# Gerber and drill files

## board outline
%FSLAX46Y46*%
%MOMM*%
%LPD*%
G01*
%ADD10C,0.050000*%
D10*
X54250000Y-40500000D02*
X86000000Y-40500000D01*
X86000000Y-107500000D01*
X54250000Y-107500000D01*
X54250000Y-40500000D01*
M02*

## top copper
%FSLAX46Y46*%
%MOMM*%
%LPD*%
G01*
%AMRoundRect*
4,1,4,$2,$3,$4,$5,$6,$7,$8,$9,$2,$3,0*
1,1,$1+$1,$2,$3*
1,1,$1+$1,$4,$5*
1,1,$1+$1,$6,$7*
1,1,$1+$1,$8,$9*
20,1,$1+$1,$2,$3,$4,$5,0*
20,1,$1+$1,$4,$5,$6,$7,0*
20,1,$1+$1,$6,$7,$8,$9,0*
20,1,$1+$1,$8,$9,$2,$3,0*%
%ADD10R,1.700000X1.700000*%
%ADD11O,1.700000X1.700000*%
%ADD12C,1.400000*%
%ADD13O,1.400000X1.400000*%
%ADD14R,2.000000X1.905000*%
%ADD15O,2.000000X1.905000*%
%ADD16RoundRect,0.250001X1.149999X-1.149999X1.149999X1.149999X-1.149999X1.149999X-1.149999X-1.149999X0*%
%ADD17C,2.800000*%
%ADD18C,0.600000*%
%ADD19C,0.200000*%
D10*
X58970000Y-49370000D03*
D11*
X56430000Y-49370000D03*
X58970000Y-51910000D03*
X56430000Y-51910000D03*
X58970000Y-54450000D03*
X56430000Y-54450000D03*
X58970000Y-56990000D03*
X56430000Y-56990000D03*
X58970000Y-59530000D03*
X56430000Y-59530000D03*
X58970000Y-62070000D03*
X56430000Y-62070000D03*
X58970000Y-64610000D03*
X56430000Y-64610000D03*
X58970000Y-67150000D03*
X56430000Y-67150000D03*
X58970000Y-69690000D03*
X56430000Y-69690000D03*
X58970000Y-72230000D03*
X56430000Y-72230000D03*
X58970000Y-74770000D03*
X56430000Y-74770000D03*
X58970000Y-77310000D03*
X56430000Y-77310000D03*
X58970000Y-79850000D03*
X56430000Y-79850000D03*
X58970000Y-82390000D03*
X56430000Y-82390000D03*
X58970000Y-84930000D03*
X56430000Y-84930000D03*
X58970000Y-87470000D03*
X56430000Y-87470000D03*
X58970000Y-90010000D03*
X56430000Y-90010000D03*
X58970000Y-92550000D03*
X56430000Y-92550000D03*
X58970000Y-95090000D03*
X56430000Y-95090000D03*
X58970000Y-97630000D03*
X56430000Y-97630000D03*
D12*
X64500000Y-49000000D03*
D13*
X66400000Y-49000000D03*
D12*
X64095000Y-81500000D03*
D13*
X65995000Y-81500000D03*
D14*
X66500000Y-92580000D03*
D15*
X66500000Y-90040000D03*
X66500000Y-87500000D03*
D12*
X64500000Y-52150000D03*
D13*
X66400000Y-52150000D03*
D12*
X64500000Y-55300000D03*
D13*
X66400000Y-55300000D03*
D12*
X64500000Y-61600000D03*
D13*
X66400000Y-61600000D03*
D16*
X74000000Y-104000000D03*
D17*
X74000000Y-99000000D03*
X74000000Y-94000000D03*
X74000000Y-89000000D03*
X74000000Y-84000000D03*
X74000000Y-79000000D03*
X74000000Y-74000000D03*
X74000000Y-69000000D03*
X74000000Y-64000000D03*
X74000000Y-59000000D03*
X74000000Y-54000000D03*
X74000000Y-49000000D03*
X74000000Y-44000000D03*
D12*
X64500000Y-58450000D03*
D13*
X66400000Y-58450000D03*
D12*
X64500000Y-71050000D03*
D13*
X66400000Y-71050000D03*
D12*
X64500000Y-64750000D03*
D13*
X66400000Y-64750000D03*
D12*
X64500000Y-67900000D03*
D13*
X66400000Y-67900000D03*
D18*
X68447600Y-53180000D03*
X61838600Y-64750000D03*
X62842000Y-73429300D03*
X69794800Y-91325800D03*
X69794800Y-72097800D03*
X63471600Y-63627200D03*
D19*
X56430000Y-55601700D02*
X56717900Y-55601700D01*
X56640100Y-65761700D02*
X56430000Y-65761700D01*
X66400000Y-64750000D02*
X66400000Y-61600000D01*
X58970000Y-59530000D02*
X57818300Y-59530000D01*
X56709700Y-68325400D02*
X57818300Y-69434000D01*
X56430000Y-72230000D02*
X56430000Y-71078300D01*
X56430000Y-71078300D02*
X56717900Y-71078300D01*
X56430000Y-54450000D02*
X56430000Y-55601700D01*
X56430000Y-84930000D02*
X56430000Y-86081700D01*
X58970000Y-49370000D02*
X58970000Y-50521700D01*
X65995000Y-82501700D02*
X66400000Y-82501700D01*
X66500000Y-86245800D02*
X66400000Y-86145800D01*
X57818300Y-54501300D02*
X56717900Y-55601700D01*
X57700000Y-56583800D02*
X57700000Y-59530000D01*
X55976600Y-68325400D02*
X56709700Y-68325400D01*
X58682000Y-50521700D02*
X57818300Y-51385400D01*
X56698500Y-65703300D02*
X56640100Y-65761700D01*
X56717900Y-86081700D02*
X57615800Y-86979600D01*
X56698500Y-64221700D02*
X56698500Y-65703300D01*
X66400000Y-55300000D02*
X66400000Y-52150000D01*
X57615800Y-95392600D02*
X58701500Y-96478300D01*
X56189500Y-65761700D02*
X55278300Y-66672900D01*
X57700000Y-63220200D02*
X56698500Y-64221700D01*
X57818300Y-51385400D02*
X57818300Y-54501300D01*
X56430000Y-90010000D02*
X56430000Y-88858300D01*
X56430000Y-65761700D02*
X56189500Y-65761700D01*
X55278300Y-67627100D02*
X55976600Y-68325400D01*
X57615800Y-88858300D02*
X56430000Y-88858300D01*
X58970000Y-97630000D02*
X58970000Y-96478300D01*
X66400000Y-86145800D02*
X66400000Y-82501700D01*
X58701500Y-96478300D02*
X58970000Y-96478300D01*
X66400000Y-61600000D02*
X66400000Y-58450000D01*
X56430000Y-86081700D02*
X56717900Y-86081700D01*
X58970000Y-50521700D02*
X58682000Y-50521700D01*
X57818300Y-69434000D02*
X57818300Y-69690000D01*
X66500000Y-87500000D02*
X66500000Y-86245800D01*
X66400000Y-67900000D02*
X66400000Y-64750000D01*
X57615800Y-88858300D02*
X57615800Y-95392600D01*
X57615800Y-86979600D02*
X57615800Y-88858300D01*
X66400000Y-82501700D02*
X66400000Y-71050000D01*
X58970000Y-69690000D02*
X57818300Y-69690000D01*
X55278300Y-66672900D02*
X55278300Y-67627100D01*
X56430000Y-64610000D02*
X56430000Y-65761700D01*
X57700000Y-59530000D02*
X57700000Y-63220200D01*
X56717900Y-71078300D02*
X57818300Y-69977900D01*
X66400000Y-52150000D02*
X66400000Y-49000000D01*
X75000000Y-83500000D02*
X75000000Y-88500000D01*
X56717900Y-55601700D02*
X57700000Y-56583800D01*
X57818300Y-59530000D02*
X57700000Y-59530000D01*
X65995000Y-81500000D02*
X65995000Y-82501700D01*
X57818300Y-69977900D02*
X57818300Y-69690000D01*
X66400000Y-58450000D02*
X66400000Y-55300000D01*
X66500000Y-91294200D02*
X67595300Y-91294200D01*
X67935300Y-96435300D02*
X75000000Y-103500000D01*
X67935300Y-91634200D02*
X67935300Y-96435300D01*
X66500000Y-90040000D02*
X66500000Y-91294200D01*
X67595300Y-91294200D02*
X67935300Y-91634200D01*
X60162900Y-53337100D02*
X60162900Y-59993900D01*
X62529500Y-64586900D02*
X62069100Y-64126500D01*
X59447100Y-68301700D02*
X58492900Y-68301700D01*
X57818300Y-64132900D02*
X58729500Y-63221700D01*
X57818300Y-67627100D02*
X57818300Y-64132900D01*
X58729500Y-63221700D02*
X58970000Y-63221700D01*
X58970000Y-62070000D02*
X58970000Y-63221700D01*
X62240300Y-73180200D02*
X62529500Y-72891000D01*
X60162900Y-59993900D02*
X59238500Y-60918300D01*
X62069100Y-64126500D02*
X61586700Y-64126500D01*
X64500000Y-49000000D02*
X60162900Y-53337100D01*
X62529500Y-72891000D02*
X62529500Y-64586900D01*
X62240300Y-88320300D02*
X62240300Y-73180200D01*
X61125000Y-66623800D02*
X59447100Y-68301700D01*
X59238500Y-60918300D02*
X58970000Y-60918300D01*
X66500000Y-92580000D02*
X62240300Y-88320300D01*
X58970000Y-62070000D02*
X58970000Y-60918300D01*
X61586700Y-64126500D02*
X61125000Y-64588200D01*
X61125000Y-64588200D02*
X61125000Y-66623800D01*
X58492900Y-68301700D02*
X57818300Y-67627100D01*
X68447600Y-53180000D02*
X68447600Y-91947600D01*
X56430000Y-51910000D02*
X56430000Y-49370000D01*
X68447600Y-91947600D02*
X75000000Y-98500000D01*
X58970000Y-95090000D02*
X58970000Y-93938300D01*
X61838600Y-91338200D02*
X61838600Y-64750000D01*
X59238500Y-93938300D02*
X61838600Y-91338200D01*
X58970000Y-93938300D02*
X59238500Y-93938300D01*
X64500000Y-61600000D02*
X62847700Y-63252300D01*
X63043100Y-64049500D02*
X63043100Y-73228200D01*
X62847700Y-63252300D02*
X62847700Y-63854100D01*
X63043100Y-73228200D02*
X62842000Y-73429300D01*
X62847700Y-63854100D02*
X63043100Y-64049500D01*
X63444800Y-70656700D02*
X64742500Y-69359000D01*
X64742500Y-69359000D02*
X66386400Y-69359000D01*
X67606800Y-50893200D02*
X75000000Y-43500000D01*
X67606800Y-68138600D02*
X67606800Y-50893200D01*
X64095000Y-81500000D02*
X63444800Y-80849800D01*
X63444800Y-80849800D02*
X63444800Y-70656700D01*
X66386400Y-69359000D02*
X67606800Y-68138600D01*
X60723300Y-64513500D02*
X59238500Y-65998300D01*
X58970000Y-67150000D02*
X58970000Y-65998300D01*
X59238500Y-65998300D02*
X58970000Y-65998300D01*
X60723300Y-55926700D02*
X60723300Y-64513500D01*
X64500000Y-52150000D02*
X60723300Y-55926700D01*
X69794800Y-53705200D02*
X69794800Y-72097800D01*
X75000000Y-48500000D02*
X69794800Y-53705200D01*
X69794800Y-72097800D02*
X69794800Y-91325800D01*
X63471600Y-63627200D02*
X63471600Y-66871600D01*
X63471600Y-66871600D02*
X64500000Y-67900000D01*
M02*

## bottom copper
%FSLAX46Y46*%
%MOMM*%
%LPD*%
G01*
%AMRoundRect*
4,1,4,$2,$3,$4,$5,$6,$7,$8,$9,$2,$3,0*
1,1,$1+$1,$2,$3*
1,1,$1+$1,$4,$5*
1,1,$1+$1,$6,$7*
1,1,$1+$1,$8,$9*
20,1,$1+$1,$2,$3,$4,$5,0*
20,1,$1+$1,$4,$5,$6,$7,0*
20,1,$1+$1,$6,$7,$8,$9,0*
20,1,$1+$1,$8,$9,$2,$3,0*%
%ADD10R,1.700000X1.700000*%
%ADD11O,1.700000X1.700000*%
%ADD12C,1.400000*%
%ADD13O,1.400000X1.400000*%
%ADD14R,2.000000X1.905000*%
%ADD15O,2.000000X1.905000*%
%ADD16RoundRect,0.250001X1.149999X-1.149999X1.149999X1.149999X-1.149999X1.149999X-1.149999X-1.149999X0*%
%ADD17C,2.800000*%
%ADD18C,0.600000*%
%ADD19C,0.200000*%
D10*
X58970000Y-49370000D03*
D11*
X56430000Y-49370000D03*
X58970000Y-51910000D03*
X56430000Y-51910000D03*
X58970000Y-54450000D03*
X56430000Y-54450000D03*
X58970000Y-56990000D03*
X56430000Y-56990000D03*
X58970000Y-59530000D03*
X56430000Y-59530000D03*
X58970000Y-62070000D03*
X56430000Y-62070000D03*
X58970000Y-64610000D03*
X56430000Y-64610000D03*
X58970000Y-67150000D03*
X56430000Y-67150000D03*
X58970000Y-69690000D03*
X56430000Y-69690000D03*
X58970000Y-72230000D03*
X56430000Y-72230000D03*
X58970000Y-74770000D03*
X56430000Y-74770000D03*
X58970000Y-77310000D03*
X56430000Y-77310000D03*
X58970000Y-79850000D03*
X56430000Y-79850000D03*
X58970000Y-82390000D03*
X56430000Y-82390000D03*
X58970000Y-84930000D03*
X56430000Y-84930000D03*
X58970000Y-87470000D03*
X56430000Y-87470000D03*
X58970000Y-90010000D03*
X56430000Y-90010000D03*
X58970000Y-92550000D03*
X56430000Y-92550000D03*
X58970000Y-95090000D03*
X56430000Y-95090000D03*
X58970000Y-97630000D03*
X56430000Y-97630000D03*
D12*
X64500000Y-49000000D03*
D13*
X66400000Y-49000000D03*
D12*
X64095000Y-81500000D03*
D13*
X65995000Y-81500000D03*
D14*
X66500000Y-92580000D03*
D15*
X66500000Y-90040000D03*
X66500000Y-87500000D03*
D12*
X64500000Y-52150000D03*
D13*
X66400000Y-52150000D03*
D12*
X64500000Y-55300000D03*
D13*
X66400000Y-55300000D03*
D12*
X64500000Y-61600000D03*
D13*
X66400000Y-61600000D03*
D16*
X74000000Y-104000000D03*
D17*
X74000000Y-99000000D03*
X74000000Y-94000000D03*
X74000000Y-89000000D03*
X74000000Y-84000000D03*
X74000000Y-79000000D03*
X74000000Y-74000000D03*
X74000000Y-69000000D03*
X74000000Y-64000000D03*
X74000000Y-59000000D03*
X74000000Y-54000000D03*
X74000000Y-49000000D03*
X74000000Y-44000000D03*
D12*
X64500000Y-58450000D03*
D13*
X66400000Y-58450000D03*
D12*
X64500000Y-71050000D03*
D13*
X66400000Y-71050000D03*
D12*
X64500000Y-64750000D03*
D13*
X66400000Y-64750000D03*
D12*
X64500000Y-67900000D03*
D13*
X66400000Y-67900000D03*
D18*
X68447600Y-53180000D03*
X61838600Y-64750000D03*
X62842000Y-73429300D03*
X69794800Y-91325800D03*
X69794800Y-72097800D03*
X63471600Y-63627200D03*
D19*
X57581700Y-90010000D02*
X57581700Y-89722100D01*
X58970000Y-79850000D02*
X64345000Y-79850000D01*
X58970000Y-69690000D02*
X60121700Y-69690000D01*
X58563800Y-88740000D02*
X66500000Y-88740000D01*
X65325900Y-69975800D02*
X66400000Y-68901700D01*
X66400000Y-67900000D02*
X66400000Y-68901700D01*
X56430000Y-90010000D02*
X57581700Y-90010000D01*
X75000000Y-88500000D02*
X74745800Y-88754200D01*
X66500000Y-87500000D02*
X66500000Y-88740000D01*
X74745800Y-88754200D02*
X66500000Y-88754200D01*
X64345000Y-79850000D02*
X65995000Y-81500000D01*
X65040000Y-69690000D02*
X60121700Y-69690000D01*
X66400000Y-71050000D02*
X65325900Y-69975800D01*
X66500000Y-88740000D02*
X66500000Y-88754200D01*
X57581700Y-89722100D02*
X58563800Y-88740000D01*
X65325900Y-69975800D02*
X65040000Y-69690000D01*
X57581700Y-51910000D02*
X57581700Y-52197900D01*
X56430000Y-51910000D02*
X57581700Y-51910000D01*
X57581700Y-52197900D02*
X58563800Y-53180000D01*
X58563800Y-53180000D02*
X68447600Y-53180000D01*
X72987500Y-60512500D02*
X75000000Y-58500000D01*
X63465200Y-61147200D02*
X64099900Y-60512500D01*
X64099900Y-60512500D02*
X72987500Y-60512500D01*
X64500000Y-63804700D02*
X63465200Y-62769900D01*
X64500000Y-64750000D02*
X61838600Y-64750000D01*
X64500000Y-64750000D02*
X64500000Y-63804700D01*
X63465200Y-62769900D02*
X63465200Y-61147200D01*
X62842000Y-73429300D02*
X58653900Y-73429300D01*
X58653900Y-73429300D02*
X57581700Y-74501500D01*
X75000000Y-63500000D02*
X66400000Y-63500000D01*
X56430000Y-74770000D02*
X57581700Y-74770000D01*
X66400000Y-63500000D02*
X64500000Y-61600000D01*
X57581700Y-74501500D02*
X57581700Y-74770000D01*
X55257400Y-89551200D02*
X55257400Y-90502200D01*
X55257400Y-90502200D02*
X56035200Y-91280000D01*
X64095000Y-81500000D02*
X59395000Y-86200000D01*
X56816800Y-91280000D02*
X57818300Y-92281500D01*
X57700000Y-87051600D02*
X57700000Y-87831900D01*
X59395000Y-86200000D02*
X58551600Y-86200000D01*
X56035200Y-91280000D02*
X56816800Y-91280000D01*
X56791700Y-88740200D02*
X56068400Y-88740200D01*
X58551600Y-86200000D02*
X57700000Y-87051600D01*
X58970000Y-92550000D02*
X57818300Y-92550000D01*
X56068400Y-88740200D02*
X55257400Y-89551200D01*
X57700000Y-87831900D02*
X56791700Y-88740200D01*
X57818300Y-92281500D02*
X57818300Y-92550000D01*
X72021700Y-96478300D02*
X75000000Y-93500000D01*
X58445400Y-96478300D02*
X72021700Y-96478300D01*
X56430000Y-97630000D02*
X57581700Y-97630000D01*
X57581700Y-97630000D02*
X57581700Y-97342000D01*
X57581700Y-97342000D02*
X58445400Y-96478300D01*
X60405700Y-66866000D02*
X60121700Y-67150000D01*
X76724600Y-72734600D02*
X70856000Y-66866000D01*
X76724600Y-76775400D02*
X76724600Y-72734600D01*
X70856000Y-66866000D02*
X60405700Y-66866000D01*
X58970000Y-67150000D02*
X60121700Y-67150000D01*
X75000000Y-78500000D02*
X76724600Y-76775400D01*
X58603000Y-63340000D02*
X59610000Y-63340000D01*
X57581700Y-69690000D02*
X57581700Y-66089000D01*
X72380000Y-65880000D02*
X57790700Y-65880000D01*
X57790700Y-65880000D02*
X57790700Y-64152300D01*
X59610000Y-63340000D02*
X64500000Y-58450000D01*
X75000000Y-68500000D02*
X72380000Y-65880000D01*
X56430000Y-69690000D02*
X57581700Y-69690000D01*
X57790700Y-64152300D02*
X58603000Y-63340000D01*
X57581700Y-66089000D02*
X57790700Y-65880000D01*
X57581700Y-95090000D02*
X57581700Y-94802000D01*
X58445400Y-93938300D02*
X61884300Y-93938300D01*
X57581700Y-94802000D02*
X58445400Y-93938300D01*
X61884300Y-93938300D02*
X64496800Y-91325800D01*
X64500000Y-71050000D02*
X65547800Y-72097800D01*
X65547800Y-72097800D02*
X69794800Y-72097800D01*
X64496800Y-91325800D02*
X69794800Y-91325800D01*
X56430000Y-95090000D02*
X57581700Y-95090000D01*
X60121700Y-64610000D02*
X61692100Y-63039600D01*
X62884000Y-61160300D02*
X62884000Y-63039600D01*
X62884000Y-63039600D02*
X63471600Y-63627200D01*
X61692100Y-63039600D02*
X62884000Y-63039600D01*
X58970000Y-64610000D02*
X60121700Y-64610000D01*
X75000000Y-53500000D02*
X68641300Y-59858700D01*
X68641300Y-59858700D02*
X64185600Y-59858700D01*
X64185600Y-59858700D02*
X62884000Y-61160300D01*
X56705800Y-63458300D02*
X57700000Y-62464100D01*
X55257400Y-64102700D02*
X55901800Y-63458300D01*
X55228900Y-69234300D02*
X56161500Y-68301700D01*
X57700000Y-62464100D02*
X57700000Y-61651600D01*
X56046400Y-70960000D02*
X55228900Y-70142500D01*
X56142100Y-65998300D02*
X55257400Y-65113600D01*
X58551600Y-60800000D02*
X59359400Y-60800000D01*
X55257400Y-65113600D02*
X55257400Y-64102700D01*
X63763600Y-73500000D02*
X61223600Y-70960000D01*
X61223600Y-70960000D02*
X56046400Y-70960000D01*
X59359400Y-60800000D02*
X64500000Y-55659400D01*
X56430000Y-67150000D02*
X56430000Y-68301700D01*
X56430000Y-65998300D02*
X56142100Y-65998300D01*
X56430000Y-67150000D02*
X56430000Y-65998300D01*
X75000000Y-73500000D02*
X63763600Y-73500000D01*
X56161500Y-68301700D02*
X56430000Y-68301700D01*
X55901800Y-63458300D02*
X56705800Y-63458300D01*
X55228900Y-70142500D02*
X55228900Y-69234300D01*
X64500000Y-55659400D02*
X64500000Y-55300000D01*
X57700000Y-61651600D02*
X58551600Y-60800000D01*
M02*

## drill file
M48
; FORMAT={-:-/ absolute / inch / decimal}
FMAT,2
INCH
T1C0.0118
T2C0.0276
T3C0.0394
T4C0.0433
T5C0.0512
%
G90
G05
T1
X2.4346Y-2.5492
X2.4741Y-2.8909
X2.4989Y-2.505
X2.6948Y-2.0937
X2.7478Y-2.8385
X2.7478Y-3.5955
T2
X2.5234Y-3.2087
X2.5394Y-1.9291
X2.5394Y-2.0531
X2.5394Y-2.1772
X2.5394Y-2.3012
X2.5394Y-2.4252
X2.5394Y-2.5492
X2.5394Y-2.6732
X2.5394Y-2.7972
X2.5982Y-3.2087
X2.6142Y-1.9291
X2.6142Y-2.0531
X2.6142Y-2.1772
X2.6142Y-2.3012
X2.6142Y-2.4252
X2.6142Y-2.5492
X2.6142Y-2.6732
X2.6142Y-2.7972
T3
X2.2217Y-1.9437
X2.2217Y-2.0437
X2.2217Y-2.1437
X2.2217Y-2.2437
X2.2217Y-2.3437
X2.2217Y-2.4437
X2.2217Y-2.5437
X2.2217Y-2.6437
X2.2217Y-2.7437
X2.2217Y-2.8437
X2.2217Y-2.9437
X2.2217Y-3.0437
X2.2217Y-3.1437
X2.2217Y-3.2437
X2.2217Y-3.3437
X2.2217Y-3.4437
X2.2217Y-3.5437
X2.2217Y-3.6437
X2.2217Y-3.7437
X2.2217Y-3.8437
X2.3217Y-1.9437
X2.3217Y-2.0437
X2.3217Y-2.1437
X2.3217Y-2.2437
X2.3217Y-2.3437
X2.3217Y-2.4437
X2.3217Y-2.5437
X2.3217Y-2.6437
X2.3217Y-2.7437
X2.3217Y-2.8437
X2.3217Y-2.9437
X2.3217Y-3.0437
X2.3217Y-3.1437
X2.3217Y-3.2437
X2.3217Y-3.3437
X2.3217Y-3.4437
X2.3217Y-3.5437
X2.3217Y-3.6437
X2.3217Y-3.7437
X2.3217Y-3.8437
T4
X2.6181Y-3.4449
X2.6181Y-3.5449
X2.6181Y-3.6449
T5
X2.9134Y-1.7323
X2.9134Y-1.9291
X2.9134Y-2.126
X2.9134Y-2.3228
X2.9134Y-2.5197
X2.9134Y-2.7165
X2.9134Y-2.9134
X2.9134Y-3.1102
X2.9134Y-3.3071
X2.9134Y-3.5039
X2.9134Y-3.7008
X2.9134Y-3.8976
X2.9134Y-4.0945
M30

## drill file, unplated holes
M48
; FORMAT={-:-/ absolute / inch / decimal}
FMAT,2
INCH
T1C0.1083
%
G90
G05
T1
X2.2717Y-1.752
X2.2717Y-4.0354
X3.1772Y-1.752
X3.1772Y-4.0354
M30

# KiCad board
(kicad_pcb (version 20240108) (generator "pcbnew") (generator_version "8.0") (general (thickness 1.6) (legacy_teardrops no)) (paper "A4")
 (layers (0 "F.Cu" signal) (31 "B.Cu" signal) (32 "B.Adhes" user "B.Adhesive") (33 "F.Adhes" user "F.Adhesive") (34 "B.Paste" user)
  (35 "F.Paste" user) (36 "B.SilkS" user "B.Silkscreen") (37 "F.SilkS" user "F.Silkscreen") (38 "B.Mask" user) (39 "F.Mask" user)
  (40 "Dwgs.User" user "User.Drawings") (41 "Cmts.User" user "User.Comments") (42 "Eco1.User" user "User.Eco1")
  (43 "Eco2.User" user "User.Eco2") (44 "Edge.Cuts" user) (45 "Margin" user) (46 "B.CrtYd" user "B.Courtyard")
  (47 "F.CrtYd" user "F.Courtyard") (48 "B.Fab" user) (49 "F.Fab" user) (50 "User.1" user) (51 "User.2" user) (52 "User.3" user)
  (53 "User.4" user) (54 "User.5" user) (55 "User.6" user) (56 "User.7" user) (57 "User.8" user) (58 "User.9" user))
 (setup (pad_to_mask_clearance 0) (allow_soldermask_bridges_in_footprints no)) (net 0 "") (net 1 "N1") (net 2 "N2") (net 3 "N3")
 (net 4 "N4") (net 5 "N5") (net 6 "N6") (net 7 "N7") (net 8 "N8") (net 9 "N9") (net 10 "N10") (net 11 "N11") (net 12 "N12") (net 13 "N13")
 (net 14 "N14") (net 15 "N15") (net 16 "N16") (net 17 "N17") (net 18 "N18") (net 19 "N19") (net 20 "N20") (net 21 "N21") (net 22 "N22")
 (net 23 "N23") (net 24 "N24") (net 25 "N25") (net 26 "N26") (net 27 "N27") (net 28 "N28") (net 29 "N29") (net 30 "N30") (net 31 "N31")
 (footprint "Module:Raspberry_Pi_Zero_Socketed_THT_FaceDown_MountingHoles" (layer "F.Cu") (at 58.97 49.37)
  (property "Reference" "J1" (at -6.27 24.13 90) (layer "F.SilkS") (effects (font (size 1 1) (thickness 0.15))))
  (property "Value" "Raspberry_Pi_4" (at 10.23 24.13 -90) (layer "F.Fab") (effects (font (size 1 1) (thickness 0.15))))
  (pad "" np_thru_hole circle (at -1.27 -4.87 90) (size 2.75 2.75) (drill 2.75) (layers "*.Cu" "*.Mask") (solder_mask_margin 1.625))
  (pad "" np_thru_hole circle (at -1.27 53.13 90) (size 2.75 2.75) (drill 2.75) (layers "*.Cu" "*.Mask") (solder_mask_margin 1.625))
  (pad "" np_thru_hole circle (at 21.73 -4.87 90) (size 2.75 2.75) (drill 2.75) (layers "*.Cu" "*.Mask") (solder_mask_margin 1.625))
  (pad "" np_thru_hole circle (at 21.73 53.13 90) (size 2.75 2.75) (drill 2.75) (layers "*.Cu" "*.Mask") (solder_mask_margin 1.625))
  (pad "1" thru_hole rect (at 0 0) (size 1.7 1.7) (drill 1) (layers "*.Cu" "*.Mask") (remove_unused_layers no) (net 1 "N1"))
  (pad "2" thru_hole oval (at -2.54 0) (size 1.7 1.7) (drill 1) (layers "*.Cu" "*.Mask") (remove_unused_layers no) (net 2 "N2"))
  (pad "3" thru_hole oval (at 0 2.54) (size 1.7 1.7) (drill 1) (layers "*.Cu" "*.Mask") (remove_unused_layers no) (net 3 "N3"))
  (pad "4" thru_hole oval (at -2.54 2.54) (size 1.7 1.7) (drill 1) (layers "*.Cu" "*.Mask") (remove_unused_layers no) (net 2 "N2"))
  (pad "5" thru_hole oval (at 0 5.08) (size 1.7 1.7) (drill 1) (layers "*.Cu" "*.Mask") (remove_unused_layers no) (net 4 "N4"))
  (pad "6" thru_hole oval (at -2.54 5.08) (size 1.7 1.7) (drill 1) (layers "*.Cu" "*.Mask") (remove_unused_layers no) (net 1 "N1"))
  (pad "7" thru_hole oval (at 0 7.62) (size 1.7 1.7) (drill 1) (layers "*.Cu" "*.Mask") (remove_unused_layers no) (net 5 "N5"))
  (pad "8" thru_hole oval (at -2.54 7.62) (size 1.7 1.7) (drill 1) (layers "*.Cu" "*.Mask") (remove_unused_layers no) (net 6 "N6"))
  (pad "9" thru_hole oval (at 0 10.16) (size 1.7 1.7) (drill 1) (layers "*.Cu" "*.Mask") (remove_unused_layers no) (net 1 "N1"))
  (pad "10" thru_hole oval (at -2.54 10.16) (size 1.7 1.7) (drill 1) (layers "*.Cu" "*.Mask") (remove_unused_layers no) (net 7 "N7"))
  (pad "11" thru_hole oval (at 0 12.7) (size 1.7 1.7) (drill 1) (layers "*.Cu" "*.Mask") (remove_unused_layers no) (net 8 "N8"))
  (pad "12" thru_hole oval (at -2.54 12.7) (size 1.7 1.7) (drill 1) (layers "*.Cu" "*.Mask") (remove_unused_layers no) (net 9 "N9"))
  (pad "13" thru_hole oval (at 0 15.24) (size 1.7 1.7) (drill 1) (layers "*.Cu" "*.Mask") (remove_unused_layers no) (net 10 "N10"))
  (pad "14" thru_hole oval (at -2.54 15.24) (size 1.7 1.7) (drill 1) (layers "*.Cu" "*.Mask") (remove_unused_layers no) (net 1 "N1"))
  (pad "15" thru_hole oval (at 0 17.78) (size 1.7 1.7) (drill 1) (layers "*.Cu" "*.Mask") (remove_unused_layers no) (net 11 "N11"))
  (pad "16" thru_hole oval (at -2.54 17.78) (size 1.7 1.7) (drill 1) (layers "*.Cu" "*.Mask") (remove_unused_layers no) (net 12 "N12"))
  (pad "17" thru_hole oval (at 0 20.32) (size 1.7 1.7) (drill 1) (layers "*.Cu" "*.Mask") (remove_unused_layers no) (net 1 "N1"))
  (pad "18" thru_hole oval (at -2.54 20.32) (size 1.7 1.7) (drill 1) (layers "*.Cu" "*.Mask") (remove_unused_layers no) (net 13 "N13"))
  (pad "19" thru_hole oval (at 0 22.86) (size 1.7 1.7) (drill 1) (layers "*.Cu" "*.Mask") (remove_unused_layers no) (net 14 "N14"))
  (pad "20" thru_hole oval (at -2.54 22.86) (size 1.7 1.7) (drill 1) (layers "*.Cu" "*.Mask") (remove_unused_layers no) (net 1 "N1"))
  (pad "21" thru_hole oval (at 0 25.4) (size 1.7 1.7) (drill 1) (layers "*.Cu" "*.Mask") (remove_unused_layers no) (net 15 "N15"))
  (pad "22" thru_hole oval (at -2.54 25.4) (size 1.7 1.7) (drill 1) (layers "*.Cu" "*.Mask") (remove_unused_layers no) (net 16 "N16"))
  (pad "23" thru_hole oval (at 0 27.94) (size 1.7 1.7) (drill 1) (layers "*.Cu" "*.Mask") (remove_unused_layers no) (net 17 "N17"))
  (pad "24" thru_hole oval (at -2.54 27.94) (size 1.7 1.7) (drill 1) (layers "*.Cu" "*.Mask") (remove_unused_layers no) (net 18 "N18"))
  (pad "25" thru_hole oval (at 0 30.48) (size 1.7 1.7) (drill 1) (layers "*.Cu" "*.Mask") (remove_unused_layers no) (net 1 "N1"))
  (pad "26" thru_hole oval (at -2.54 30.48) (size 1.7 1.7) (drill 1) (layers "*.Cu" "*.Mask") (remove_unused_layers no) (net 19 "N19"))
  (pad "27" thru_hole oval (at 0 33.02) (size 1.7 1.7) (drill 1) (layers "*.Cu" "*.Mask") (remove_unused_layers no) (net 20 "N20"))
  (pad "28" thru_hole oval (at -2.54 33.02) (size 1.7 1.7) (drill 1) (layers "*.Cu" "*.Mask") (remove_unused_layers no) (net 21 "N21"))
  (pad "29" thru_hole oval (at 0 35.56) (size 1.7 1.7) (drill 1) (layers "*.Cu" "*.Mask") (remove_unused_layers no) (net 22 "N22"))
  (pad "30" thru_hole oval (at -2.54 35.56) (size 1.7 1.7) (drill 1) (layers "*.Cu" "*.Mask") (remove_unused_layers no) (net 1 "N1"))
  (pad "31" thru_hole oval (at 0 38.1) (size 1.7 1.7) (drill 1) (layers "*.Cu" "*.Mask") (remove_unused_layers no) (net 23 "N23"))
  (pad "32" thru_hole oval (at -2.54 38.1) (size 1.7 1.7) (drill 1) (layers "*.Cu" "*.Mask") (remove_unused_layers no) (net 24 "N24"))
  (pad "33" thru_hole oval (at 0 40.64) (size 1.7 1.7) (drill 1) (layers "*.Cu" "*.Mask") (remove_unused_layers no) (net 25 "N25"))
  (pad "34" thru_hole oval (at -2.54 40.64) (size 1.7 1.7) (drill 1) (layers "*.Cu" "*.Mask") (remove_unused_layers no) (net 1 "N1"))
  (pad "35" thru_hole oval (at 0 43.18) (size 1.7 1.7) (drill 1) (layers "*.Cu" "*.Mask") (remove_unused_layers no) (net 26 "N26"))
  (pad "36" thru_hole oval (at -2.54 43.18) (size 1.7 1.7) (drill 1) (layers "*.Cu" "*.Mask") (remove_unused_layers no) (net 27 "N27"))
  (pad "37" thru_hole oval (at 0 45.72) (size 1.7 1.7) (drill 1) (layers "*.Cu" "*.Mask") (remove_unused_layers no) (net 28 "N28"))
  (pad "38" thru_hole oval (at -2.54 45.72) (size 1.7 1.7) (drill 1) (layers "*.Cu" "*.Mask") (remove_unused_layers no) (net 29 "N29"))
  (pad "39" thru_hole oval (at 0 48.26) (size 1.7 1.7) (drill 1) (layers "*.Cu" "*.Mask") (remove_unused_layers no) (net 1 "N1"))
  (pad "40" thru_hole oval (at -2.54 48.26) (size 1.7 1.7) (drill 1) (layers "*.Cu" "*.Mask") (remove_unused_layers no) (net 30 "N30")))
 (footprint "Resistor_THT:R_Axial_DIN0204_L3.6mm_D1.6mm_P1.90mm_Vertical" (layer "F.Cu") (at 64.5 49)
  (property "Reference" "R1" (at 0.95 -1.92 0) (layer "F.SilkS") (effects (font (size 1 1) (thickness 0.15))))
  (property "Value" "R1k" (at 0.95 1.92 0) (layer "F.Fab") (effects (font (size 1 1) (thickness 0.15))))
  (pad "1" thru_hole circle (at 0 0) (size 1.4 1.4) (drill 0.7) (layers "*.Cu" "*.Mask") (remove_unused_layers no) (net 8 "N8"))
  (pad "2" thru_hole oval (at 1.9 0) (size 1.4 1.4) (drill 0.7) (layers "*.Cu" "*.Mask") (remove_unused_layers no) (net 1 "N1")))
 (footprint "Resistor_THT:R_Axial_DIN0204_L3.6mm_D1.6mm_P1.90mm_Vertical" (layer "F.Cu") (at 64.095 81.5)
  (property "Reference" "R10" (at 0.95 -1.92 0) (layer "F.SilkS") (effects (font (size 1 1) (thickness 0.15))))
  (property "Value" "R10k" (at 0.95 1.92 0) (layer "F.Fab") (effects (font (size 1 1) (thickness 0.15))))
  (pad "1" thru_hole circle (at 0 0) (size 1.4 1.4) (drill 0.7) (layers "*.Cu" "*.Mask") (remove_unused_layers no) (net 26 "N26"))
  (pad "2" thru_hole oval (at 1.9 0) (size 1.4 1.4) (drill 0.7) (layers "*.Cu" "*.Mask") (remove_unused_layers no) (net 1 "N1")))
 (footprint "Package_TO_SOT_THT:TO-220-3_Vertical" (layer "F.Cu") (at 66.5 92.58 90)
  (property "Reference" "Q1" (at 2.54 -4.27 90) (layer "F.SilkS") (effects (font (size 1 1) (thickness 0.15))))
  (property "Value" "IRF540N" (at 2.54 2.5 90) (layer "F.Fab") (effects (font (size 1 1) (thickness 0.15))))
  (pad "1" thru_hole rect (at 0 0 90) (size 1.905 2) (drill 1.1) (layers "*.Cu" "*.Mask") (remove_unused_layers no) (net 8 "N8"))
  (pad "2" thru_hole oval (at 2.54 0 90) (size 1.905 2) (drill 1.1) (layers "*.Cu" "*.Mask") (remove_unused_layers no) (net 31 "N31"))
  (pad "3" thru_hole oval (at 5.08 0 90) (size 1.905 2) (drill 1.1) (layers "*.Cu" "*.Mask") (remove_unused_layers no) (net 1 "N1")))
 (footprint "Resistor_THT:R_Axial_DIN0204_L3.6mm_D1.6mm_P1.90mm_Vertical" (layer "F.Cu") (at 64.5 52.15)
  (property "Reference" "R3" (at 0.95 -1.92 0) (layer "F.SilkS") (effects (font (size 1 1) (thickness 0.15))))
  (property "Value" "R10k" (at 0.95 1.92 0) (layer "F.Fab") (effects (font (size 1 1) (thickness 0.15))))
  (pad "1" thru_hole circle (at 0 0) (size 1.4 1.4) (drill 0.7) (layers "*.Cu" "*.Mask") (remove_unused_layers no) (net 11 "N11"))
  (pad "2" thru_hole oval (at 1.9 0) (size 1.4 1.4) (drill 0.7) (layers "*.Cu" "*.Mask") (remove_unused_layers no) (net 1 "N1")))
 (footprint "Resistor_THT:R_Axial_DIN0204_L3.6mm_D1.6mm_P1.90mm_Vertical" (layer "F.Cu") (at 64.5 55.3)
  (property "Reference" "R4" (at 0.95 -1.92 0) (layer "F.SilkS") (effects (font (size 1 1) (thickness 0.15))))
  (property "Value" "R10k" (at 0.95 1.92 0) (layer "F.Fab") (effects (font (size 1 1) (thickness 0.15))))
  (pad "1" thru_hole circle (at 0 0) (size 1.4 1.4) (drill 0.7) (layers "*.Cu" "*.Mask") (remove_unused_layers no) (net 12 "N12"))
  (pad "2" thru_hole oval (at 1.9 0) (size 1.4 1.4) (drill 0.7) (layers "*.Cu" "*.Mask") (remove_unused_layers no) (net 1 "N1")))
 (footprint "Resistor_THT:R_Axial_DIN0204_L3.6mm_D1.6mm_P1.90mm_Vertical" (layer "F.Cu") (at 64.5 61.6)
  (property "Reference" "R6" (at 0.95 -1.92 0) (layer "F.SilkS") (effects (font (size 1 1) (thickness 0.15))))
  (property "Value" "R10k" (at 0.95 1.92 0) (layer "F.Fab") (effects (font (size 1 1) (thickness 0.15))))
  (pad "1" thru_hole circle (at 0 0) (size 1.4 1.4) (drill 0.7) (layers "*.Cu" "*.Mask") (remove_unused_layers no) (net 16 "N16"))
  (pad "2" thru_hole oval (at 1.9 0) (size 1.4 1.4) (drill 0.7) (layers "*.Cu" "*.Mask") (remove_unused_layers no) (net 1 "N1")))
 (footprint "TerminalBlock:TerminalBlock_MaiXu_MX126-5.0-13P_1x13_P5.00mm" (layer "F.Cu") (at 74 104 90)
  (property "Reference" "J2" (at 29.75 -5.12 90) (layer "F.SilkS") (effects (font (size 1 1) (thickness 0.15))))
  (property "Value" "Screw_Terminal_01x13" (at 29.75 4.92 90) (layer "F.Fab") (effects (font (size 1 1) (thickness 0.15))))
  (pad "1" thru_hole roundrect (at 0 0 90) (size 2.8 2.8) (drill 1.3) (layers "*.Cu" "*.Mask") (remove_unused_layers no)
   (roundrect_rratio 0.089286) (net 31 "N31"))
  (pad "2" thru_hole circle (at 5 0 90) (size 2.8 2.8) (drill 1.3) (layers "*.Cu" "*.Mask") (remove_unused_layers no) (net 2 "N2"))
  (pad "3" thru_hole circle (at 10 0 90) (size 2.8 2.8) (drill 1.3) (layers "*.Cu" "*.Mask") (remove_unused_layers no) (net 30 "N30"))
  (pad "4" thru_hole circle (at 15 0 90) (size 2.8 2.8) (drill 1.3) (layers "*.Cu" "*.Mask") (remove_unused_layers no) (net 1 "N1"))
  (pad "5" thru_hole circle (at 20 0 90) (size 2.8 2.8) (drill 1.3) (layers "*.Cu" "*.Mask") (remove_unused_layers no) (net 1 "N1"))
  (pad "6" thru_hole circle (at 25 0 90) (size 2.8 2.8) (drill 1.3) (layers "*.Cu" "*.Mask") (remove_unused_layers no) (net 11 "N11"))
  (pad "7" thru_hole circle (at 30 0 90) (size 2.8 2.8) (drill 1.3) (layers "*.Cu" "*.Mask") (remove_unused_layers no) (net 12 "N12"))
  (pad "8" thru_hole circle (at 35 0 90) (size 2.8 2.8) (drill 1.3) (layers "*.Cu" "*.Mask") (remove_unused_layers no) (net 13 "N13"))
  (pad "9" thru_hole circle (at 40 0 90) (size 2.8 2.8) (drill 1.3) (layers "*.Cu" "*.Mask") (remove_unused_layers no) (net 16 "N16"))
  (pad "10" thru_hole circle (at 45 0 90) (size 2.8 2.8) (drill 1.3) (layers "*.Cu" "*.Mask") (remove_unused_layers no) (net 28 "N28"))
  (pad "11" thru_hole circle (at 50 0 90) (size 2.8 2.8) (drill 1.3) (layers "*.Cu" "*.Mask") (remove_unused_layers no) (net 10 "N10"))
  (pad "12" thru_hole circle (at 55 0 90) (size 2.8 2.8) (drill 1.3) (layers "*.Cu" "*.Mask") (remove_unused_layers no) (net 29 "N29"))
  (pad "13" thru_hole circle (at 60 0 90) (size 2.8 2.8) (drill 1.3) (layers "*.Cu" "*.Mask") (remove_unused_layers no) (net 26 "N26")))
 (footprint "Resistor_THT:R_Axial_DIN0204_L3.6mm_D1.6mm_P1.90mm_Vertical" (layer "F.Cu") (at 64.5 58.45)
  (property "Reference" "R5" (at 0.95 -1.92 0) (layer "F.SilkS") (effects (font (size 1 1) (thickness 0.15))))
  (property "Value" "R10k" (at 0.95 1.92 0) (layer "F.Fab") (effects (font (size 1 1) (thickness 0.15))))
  (pad "1" thru_hole circle (at 0 0) (size 1.4 1.4) (drill 0.7) (layers "*.Cu" "*.Mask") (remove_unused_layers no) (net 13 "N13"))
  (pad "2" thru_hole oval (at 1.9 0) (size 1.4 1.4) (drill 0.7) (layers "*.Cu" "*.Mask") (remove_unused_layers no) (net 1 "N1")))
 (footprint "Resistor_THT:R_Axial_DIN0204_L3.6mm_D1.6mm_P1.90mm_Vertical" (layer "F.Cu") (at 64.5 71.05)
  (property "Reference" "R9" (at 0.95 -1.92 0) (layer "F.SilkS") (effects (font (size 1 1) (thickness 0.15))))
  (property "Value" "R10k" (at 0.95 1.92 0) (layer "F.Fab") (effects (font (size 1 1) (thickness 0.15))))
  (pad "1" thru_hole circle (at 0 0) (size 1.4 1.4) (drill 0.7) (layers "*.Cu" "*.Mask") (remove_unused_layers no) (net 29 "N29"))
  (pad "2" thru_hole oval (at 1.9 0) (size 1.4 1.4) (drill 0.7) (layers "*.Cu" "*.Mask") (remove_unused_layers no) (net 1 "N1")))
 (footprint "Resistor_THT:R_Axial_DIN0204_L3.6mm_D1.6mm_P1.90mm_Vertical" (layer "F.Cu") (at 64.5 64.75)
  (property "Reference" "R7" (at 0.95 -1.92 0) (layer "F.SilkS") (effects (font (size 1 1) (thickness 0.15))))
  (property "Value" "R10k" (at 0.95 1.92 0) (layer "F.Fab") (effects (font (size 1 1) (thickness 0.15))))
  (pad "1" thru_hole circle (at 0 0) (size 1.4 1.4) (drill 0.7) (layers "*.Cu" "*.Mask") (remove_unused_layers no) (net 28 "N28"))
  (pad "2" thru_hole oval (at 1.9 0) (size 1.4 1.4) (drill 0.7) (layers "*.Cu" "*.Mask") (remove_unused_layers no) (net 1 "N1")))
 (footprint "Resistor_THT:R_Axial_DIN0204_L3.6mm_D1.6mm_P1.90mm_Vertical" (layer "F.Cu") (at 64.5 67.9)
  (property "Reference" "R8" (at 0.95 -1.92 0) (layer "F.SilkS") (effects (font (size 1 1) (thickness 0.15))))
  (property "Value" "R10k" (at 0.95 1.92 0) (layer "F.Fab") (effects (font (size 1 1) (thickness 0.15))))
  (pad "1" thru_hole circle (at 0 0) (size 1.4 1.4) (drill 0.7) (layers "*.Cu" "*.Mask") (remove_unused_layers no) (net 10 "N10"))
  (pad "2" thru_hole oval (at 1.9 0) (size 1.4 1.4) (drill 0.7) (layers "*.Cu" "*.Mask") (remove_unused_layers no) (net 1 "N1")))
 (gr_rect (start 54.25 40.5) (end 86 107.5) (stroke (width 0.05) (type default)) (fill none) (layer "Edge.Cuts"))
 (segment (start 56.43 55.6017) (end 56.7179 55.6017) (width 0.2) (layer "F.Cu") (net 1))
 (segment (start 56.6401 65.7617) (end 56.43 65.7617) (width 0.2) (layer "F.Cu") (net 1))
 (segment (start 66.4 64.75) (end 66.4 61.6) (width 0.2) (layer "F.Cu") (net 1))
 (segment (start 58.97 59.53) (end 57.8183 59.53) (width 0.2) (layer "F.Cu") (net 1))
 (segment (start 56.7097 68.3254) (end 57.8183 69.434) (width 0.2) (layer "F.Cu") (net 1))
 (segment (start 56.43 72.23) (end 56.43 71.0783) (width 0.2) (layer "F.Cu") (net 1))
 (segment (start 56.43 71.0783) (end 56.7179 71.0783) (width 0.2) (layer "F.Cu") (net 1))
 (segment (start 56.43 54.45) (end 56.43 55.6017) (width 0.2) (layer "F.Cu") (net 1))
 (segment (start 56.43 84.93) (end 56.43 86.0817) (width 0.2) (layer "F.Cu") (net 1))
 (segment (start 58.97 49.37) (end 58.97 50.5217) (width 0.2) (layer "F.Cu") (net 1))
 (segment (start 65.995 82.5017) (end 66.4 82.5017) (width 0.2) (layer "F.Cu") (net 1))
 (segment (start 66.5 86.2458) (end 66.4 86.1458) (width 0.2) (layer "F.Cu") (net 1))
 (segment (start 57.8183 54.5013) (end 56.7179 55.6017) (width 0.2) (layer "F.Cu") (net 1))
 (segment (start 57.7 56.5838) (end 57.7 59.53) (width 0.2) (layer "F.Cu") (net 1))
 (segment (start 55.9766 68.3254) (end 56.7097 68.3254) (width 0.2) (layer "F.Cu") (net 1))
 (segment (start 58.682 50.5217) (end 57.8183 51.3854) (width 0.2) (layer "F.Cu") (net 1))
 (segment (start 56.6985 65.7033) (end 56.6401 65.7617) (width 0.2) (layer "F.Cu") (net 1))
 (segment (start 56.7179 86.0817) (end 57.6158 86.9796) (width 0.2) (layer "F.Cu") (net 1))
 (segment (start 56.6985 64.2217) (end 56.6985 65.7033) (width 0.2) (layer "F.Cu") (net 1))
 (segment (start 66.4 55.3) (end 66.4 52.15) (width 0.2) (layer "F.Cu") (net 1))
 (segment (start 57.6158 95.3926) (end 58.7015 96.4783) (width 0.2) (layer "F.Cu") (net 1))
 (segment (start 56.1895 65.7617) (end 55.2783 66.6729) (width 0.2) (layer "F.Cu") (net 1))
 (segment (start 57.7 63.2202) (end 56.6985 64.2217) (width 0.2) (layer "F.Cu") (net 1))
 (segment (start 57.8183 51.3854) (end 57.8183 54.5013) (width 0.2) (layer "F.Cu") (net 1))
 (segment (start 56.43 90.01) (end 56.43 88.8583) (width 0.2) (layer "F.Cu") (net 1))
 (segment (start 56.43 65.7617) (end 56.1895 65.7617) (width 0.2) (layer "F.Cu") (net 1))
 (segment (start 55.2783 67.6271) (end 55.9766 68.3254) (width 0.2) (layer "F.Cu") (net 1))
 (segment (start 57.6158 88.8583) (end 56.43 88.8583) (width 0.2) (layer "F.Cu") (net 1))
 (segment (start 58.97 97.63) (end 58.97 96.4783) (width 0.2) (layer "F.Cu") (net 1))
 (segment (start 66.4 86.1458) (end 66.4 82.5017) (width 0.2) (layer "F.Cu") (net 1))
 (segment (start 58.7015 96.4783) (end 58.97 96.4783) (width 0.2) (layer "F.Cu") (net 1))
 (segment (start 66.4 61.6) (end 66.4 58.45) (width 0.2) (layer "F.Cu") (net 1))
 (segment (start 56.43 86.0817) (end 56.7179 86.0817) (width 0.2) (layer "F.Cu") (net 1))
 (segment (start 58.97 50.5217) (end 58.682 50.5217) (width 0.2) (layer "F.Cu") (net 1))
 (segment (start 57.8183 69.434) (end 57.8183 69.69) (width 0.2) (layer "F.Cu") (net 1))
 (segment (start 66.5 87.5) (end 66.5 86.2458) (width 0.2) (layer "F.Cu") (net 1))
 (segment (start 66.4 67.9) (end 66.4 64.75) (width 0.2) (layer "F.Cu") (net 1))
 (segment (start 57.6158 88.8583) (end 57.6158 95.3926) (width 0.2) (layer "F.Cu") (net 1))
 (segment (start 57.6158 86.9796) (end 57.6158 88.8583) (width 0.2) (layer "F.Cu") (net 1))
 (segment (start 66.4 82.5017) (end 66.4 71.05) (width 0.2) (layer "F.Cu") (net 1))
 (segment (start 58.97 69.69) (end 57.8183 69.69) (width 0.2) (layer "F.Cu") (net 1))
 (segment (start 55.2783 66.6729) (end 55.2783 67.6271) (width 0.2) (layer "F.Cu") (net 1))
 (segment (start 56.43 64.61) (end 56.43 65.7617) (width 0.2) (layer "F.Cu") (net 1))
 (segment (start 57.7 59.53) (end 57.7 63.2202) (width 0.2) (layer "F.Cu") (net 1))
 (segment (start 56.7179 71.0783) (end 57.8183 69.9779) (width 0.2) (layer "F.Cu") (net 1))
 (segment (start 66.4 52.15) (end 66.4 49) (width 0.2) (layer "F.Cu") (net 1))
 (segment (start 75 83.5) (end 75 88.5) (width 0.2) (layer "F.Cu") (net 1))
 (segment (start 56.7179 55.6017) (end 57.7 56.5838) (width 0.2) (layer "F.Cu") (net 1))
 (segment (start 57.8183 59.53) (end 57.7 59.53) (width 0.2) (layer "F.Cu") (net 1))
 (segment (start 65.995 81.5) (end 65.995 82.5017) (width 0.2) (layer "F.Cu") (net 1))
 (segment (start 57.8183 69.9779) (end 57.8183 69.69) (width 0.2) (layer "F.Cu") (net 1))
 (segment (start 66.4 58.45) (end 66.4 55.3) (width 0.2) (layer "F.Cu") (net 1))
 (segment (start 57.5817 90.01) (end 57.5817 89.7221) (width 0.2) (layer "B.Cu") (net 1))
 (segment (start 58.97 79.85) (end 64.345 79.85) (width 0.2) (layer "B.Cu") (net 1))
 (segment (start 58.97 69.69) (end 60.1217 69.69) (width 0.2) (layer "B.Cu") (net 1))
 (segment (start 58.5638 88.74) (end 66.5 88.74) (width 0.2) (layer "B.Cu") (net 1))
 (segment (start 65.3259 69.9758) (end 66.4 68.9017) (width 0.2) (layer "B.Cu") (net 1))
 (segment (start 66.4 67.9) (end 66.4 68.9017) (width 0.2) (layer "B.Cu") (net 1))
 (segment (start 56.43 90.01) (end 57.5817 90.01) (width 0.2) (layer "B.Cu") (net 1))
 (segment (start 75 88.5) (end 74.7458 88.7542) (width 0.2) (layer "B.Cu") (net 1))
 (segment (start 66.5 87.5) (end 66.5 88.74) (width 0.2) (layer "B.Cu") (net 1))
 (segment (start 74.7458 88.7542) (end 66.5 88.7542) (width 0.2) (layer "B.Cu") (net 1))
 (segment (start 64.345 79.85) (end 65.995 81.5) (width 0.2) (layer "B.Cu") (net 1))
 (segment (start 65.04 69.69) (end 60.1217 69.69) (width 0.2) (layer "B.Cu") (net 1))
 (segment (start 66.4 71.05) (end 65.3259 69.9758) (width 0.2) (layer "B.Cu") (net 1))
 (segment (start 66.5 88.74) (end 66.5 88.7542) (width 0.2) (layer "B.Cu") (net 1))
 (segment (start 57.5817 89.7221) (end 58.5638 88.74) (width 0.2) (layer "B.Cu") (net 1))
 (segment (start 65.3259 69.9758) (end 65.04 69.69) (width 0.2) (layer "B.Cu") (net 1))
 (segment (start 66.5 91.2942) (end 67.5953 91.2942) (width 0.2) (layer "F.Cu") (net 31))
 (segment (start 67.9353 96.4353) (end 75 103.5) (width 0.2) (layer "F.Cu") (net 31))
 (segment (start 67.9353 91.6342) (end 67.9353 96.4353) (width 0.2) (layer "F.Cu") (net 31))
 (segment (start 66.5 90.04) (end 66.5 91.2942) (width 0.2) (layer "F.Cu") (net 31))
 (segment (start 67.5953 91.2942) (end 67.9353 91.6342) (width 0.2) (layer "F.Cu") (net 31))
 (segment (start 60.1629 53.3371) (end 60.1629 59.9939) (width 0.2) (layer "F.Cu") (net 8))
 (segment (start 62.5295 64.5869) (end 62.0691 64.1265) (width 0.2) (layer "F.Cu") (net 8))
 (segment (start 59.4471 68.3017) (end 58.4929 68.3017) (width 0.2) (layer "F.Cu") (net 8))
 (segment (start 57.8183 64.1329) (end 58.7295 63.2217) (width 0.2) (layer "F.Cu") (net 8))
 (segment (start 57.8183 67.6271) (end 57.8183 64.1329) (width 0.2) (layer "F.Cu") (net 8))
 (segment (start 58.7295 63.2217) (end 58.97 63.2217) (width 0.2) (layer "F.Cu") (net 8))
 (segment (start 58.97 62.07) (end 58.97 63.2217) (width 0.2) (layer "F.Cu") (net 8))
 (segment (start 62.2403 73.1802) (end 62.5295 72.891) (width 0.2) (layer "F.Cu") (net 8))
 (segment (start 60.1629 59.9939) (end 59.2385 60.9183) (width 0.2) (layer "F.Cu") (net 8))
 (segment (start 62.0691 64.1265) (end 61.5867 64.1265) (width 0.2) (layer "F.Cu") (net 8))
 (segment (start 64.5 49) (end 60.1629 53.3371) (width 0.2) (layer "F.Cu") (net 8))
 (segment (start 62.5295 72.891) (end 62.5295 64.5869) (width 0.2) (layer "F.Cu") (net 8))
 (segment (start 62.2403 88.3203) (end 62.2403 73.1802) (width 0.2) (layer "F.Cu") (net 8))
 (segment (start 61.125 66.6238) (end 59.4471 68.3017) (width 0.2) (layer "F.Cu") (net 8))
 (segment (start 59.2385 60.9183) (end 58.97 60.9183) (width 0.2) (layer "F.Cu") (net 8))
 (segment (start 66.5 92.58) (end 62.2403 88.3203) (width 0.2) (layer "F.Cu") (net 8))
 (segment (start 58.97 62.07) (end 58.97 60.9183) (width 0.2) (layer "F.Cu") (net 8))
 (segment (start 61.5867 64.1265) (end 61.125 64.5882) (width 0.2) (layer "F.Cu") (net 8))
 (segment (start 61.125 64.5882) (end 61.125 66.6238) (width 0.2) (layer "F.Cu") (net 8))
 (segment (start 58.4929 68.3017) (end 57.8183 67.6271) (width 0.2) (layer "F.Cu") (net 8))
 (segment (start 68.4476 53.18) (end 68.4476 91.9476) (width 0.2) (layer "F.Cu") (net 2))
 (segment (start 56.43 51.91) (end 56.43 49.37) (width 0.2) (layer "F.Cu") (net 2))
 (segment (start 68.4476 91.9476) (end 75 98.5) (width 0.2) (layer "F.Cu") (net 2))
 (via (at 68.4476 53.18) (size 0.6) (drill 0.3) (layers "F.Cu" "B.Cu") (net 2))
 (segment (start 57.5817 51.91) (end 57.5817 52.1979) (width 0.2) (layer "B.Cu") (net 2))
 (segment (start 56.43 51.91) (end 57.5817 51.91) (width 0.2) (layer "B.Cu") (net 2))
 (segment (start 57.5817 52.1979) (end 58.5638 53.18) (width 0.2) (layer "B.Cu") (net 2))
 (segment (start 58.5638 53.18) (end 68.4476 53.18) (width 0.2) (layer "B.Cu") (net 2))
 (segment (start 58.97 95.09) (end 58.97 93.9383) (width 0.2) (layer "F.Cu") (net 28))
 (segment (start 61.8386 91.3382) (end 61.8386 64.75) (width 0.2) (layer "F.Cu") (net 28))
 (segment (start 59.2385 93.9383) (end 61.8386 91.3382) (width 0.2) (layer "F.Cu") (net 28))
 (segment (start 58.97 93.9383) (end 59.2385 93.9383) (width 0.2) (layer "F.Cu") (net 28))
 (via (at 61.8386 64.75) (size 0.6) (drill 0.3) (layers "F.Cu" "B.Cu") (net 28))
 (segment (start 72.9875 60.5125) (end 75 58.5) (width 0.2) (layer "B.Cu") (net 28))
 (segment (start 63.4652 61.1472) (end 64.0999 60.5125) (width 0.2) (layer "B.Cu") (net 28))
 (segment (start 64.0999 60.5125) (end 72.9875 60.5125) (width 0.2) (layer "B.Cu") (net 28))
 (segment (start 64.5 63.8047) (end 63.4652 62.7699) (width 0.2) (layer "B.Cu") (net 28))
 (segment (start 64.5 64.75) (end 61.8386 64.75) (width 0.2) (layer "B.Cu") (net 28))
 (segment (start 64.5 64.75) (end 64.5 63.8047) (width 0.2) (layer "B.Cu") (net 28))
 (segment (start 63.4652 62.7699) (end 63.4652 61.1472) (width 0.2) (layer "B.Cu") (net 28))
 (segment (start 64.5 61.6) (end 62.8477 63.2523) (width 0.2) (layer "F.Cu") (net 16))
 (segment (start 63.0431 64.0495) (end 63.0431 73.2282) (width 0.2) (layer "F.Cu") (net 16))
 (segment (start 62.8477 63.2523) (end 62.8477 63.8541) (width 0.2) (layer "F.Cu") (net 16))
 (segment (start 63.0431 73.2282) (end 62.842 73.4293) (width 0.2) (layer "F.Cu") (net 16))
 (segment (start 62.8477 63.8541) (end 63.0431 64.0495) (width 0.2) (layer "F.Cu") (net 16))
 (via (at 62.842 73.4293) (size 0.6) (drill 0.3) (layers "F.Cu" "B.Cu") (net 16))
 (segment (start 62.842 73.4293) (end 58.6539 73.4293) (width 0.2) (layer "B.Cu") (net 16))
 (segment (start 58.6539 73.4293) (end 57.5817 74.5015) (width 0.2) (layer "B.Cu") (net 16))
 (segment (start 75 63.5) (end 66.4 63.5) (width 0.2) (layer "B.Cu") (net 16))
 (segment (start 56.43 74.77) (end 57.5817 74.77) (width 0.2) (layer "B.Cu") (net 16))
 (segment (start 66.4 63.5) (end 64.5 61.6) (width 0.2) (layer "B.Cu") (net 16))
 (segment (start 57.5817 74.5015) (end 57.5817 74.77) (width 0.2) (layer "B.Cu") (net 16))
 (segment (start 63.4448 70.6567) (end 64.7425 69.359) (width 0.2) (layer "F.Cu") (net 26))
 (segment (start 64.7425 69.359) (end 66.3864 69.359) (width 0.2) (layer "F.Cu") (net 26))
 (segment (start 67.6068 50.8932) (end 75 43.5) (width 0.2) (layer "F.Cu") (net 26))
 (segment (start 67.6068 68.1386) (end 67.6068 50.8932) (width 0.2) (layer "F.Cu") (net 26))
 (segment (start 64.095 81.5) (end 63.4448 80.8498) (width 0.2) (layer "F.Cu") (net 26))
 (segment (start 63.4448 80.8498) (end 63.4448 70.6567) (width 0.2) (layer "F.Cu") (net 26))
 (segment (start 66.3864 69.359) (end 67.6068 68.1386) (width 0.2) (layer "F.Cu") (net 26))
 (segment (start 55.2574 89.5512) (end 55.2574 90.5022) (width 0.2) (layer "B.Cu") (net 26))
 (segment (start 55.2574 90.5022) (end 56.0352 91.28) (width 0.2) (layer "B.Cu") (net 26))
 (segment (start 64.095 81.5) (end 59.395 86.2) (width 0.2) (layer "B.Cu") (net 26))
 (segment (start 56.8168 91.28) (end 57.8183 92.2815) (width 0.2) (layer "B.Cu") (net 26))
 (segment (start 57.7 87.0516) (end 57.7 87.8319) (width 0.2) (layer "B.Cu") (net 26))
 (segment (start 59.395 86.2) (end 58.5516 86.2) (width 0.2) (layer "B.Cu") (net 26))
 (segment (start 56.0352 91.28) (end 56.8168 91.28) (width 0.2) (layer "B.Cu") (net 26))
 (segment (start 56.7917 88.7402) (end 56.0684 88.7402) (width 0.2) (layer "B.Cu") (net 26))
 (segment (start 58.5516 86.2) (end 57.7 87.0516) (width 0.2) (layer "B.Cu") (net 26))
 (segment (start 58.97 92.55) (end 57.8183 92.55) (width 0.2) (layer "B.Cu") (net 26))
 (segment (start 56.0684 88.7402) (end 55.2574 89.5512) (width 0.2) (layer "B.Cu") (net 26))
 (segment (start 57.7 87.8319) (end 56.7917 88.7402) (width 0.2) (layer "B.Cu") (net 26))
 (segment (start 57.8183 92.2815) (end 57.8183 92.55) (width 0.2) (layer "B.Cu") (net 26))
 (segment (start 72.0217 96.4783) (end 75 93.5) (width 0.2) (layer "B.Cu") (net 30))
 (segment (start 58.4454 96.4783) (end 72.0217 96.4783) (width 0.2) (layer "B.Cu") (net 30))
 (segment (start 56.43 97.63) (end 57.5817 97.63) (width 0.2) (layer "B.Cu") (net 30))
 (segment (start 57.5817 97.63) (end 57.5817 97.342) (width 0.2) (layer "B.Cu") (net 30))
 (segment (start 57.5817 97.342) (end 58.4454 96.4783) (width 0.2) (layer "B.Cu") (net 30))
 (segment (start 60.7233 64.5135) (end 59.2385 65.9983) (width 0.2) (layer "F.Cu") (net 11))
 (segment (start 58.97 67.15) (end 58.97 65.9983) (width 0.2) (layer "F.Cu") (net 11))
 (segment (start 59.2385 65.9983) (end 58.97 65.9983) (width 0.2) (layer "F.Cu") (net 11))
 (segment (start 60.7233 55.9267) (end 60.7233 64.5135) (width 0.2) (layer "F.Cu") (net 11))
 (segment (start 64.5 52.15) (end 60.7233 55.9267) (width 0.2) (layer "F.Cu") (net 11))
 (segment (start 60.4057 66.866) (end 60.1217 67.15) (width 0.2) (layer "B.Cu") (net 11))
 (segment (start 76.7246 72.7346) (end 70.856 66.866) (width 0.2) (layer "B.Cu") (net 11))
 (segment (start 76.7246 76.7754) (end 76.7246 72.7346) (width 0.2) (layer "B.Cu") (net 11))
 (segment (start 70.856 66.866) (end 60.4057 66.866) (width 0.2) (layer "B.Cu") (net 11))
 (segment (start 58.97 67.15) (end 60.1217 67.15) (width 0.2) (layer "B.Cu") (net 11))
 (segment (start 75 78.5) (end 76.7246 76.7754) (width 0.2) (layer "B.Cu") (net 11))
 (segment (start 58.603 63.34) (end 59.61 63.34) (width 0.2) (layer "B.Cu") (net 13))
 (segment (start 57.5817 69.69) (end 57.5817 66.089) (width 0.2) (layer "B.Cu") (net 13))
 (segment (start 72.38 65.88) (end 57.7907 65.88) (width 0.2) (layer "B.Cu") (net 13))
 (segment (start 57.7907 65.88) (end 57.7907 64.1523) (width 0.2) (layer "B.Cu") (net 13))
 (segment (start 59.61 63.34) (end 64.5 58.45) (width 0.2) (layer "B.Cu") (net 13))
 (segment (start 75 68.5) (end 72.38 65.88) (width 0.2) (layer "B.Cu") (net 13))
 (segment (start 56.43 69.69) (end 57.5817 69.69) (width 0.2) (layer "B.Cu") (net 13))
 (segment (start 57.7907 64.1523) (end 58.603 63.34) (width 0.2) (layer "B.Cu") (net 13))
 (segment (start 57.5817 66.089) (end 57.7907 65.88) (width 0.2) (layer "B.Cu") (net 13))
 (segment (start 69.7948 53.7052) (end 69.7948 72.0978) (width 0.2) (layer "F.Cu") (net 29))
 (segment (start 75 48.5) (end 69.7948 53.7052) (width 0.2) (layer "F.Cu") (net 29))
 (segment (start 69.7948 72.0978) (end 69.7948 91.3258) (width 0.2) (layer "F.Cu") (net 29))
 (via (at 69.7948 91.3258) (size 0.6) (drill 0.3) (layers "F.Cu" "B.Cu") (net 29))
 (via (at 69.7948 72.0978) (size 0.6) (drill 0.3) (layers "F.Cu" "B.Cu") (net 29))
 (segment (start 57.5817 95.09) (end 57.5817 94.802) (width 0.2) (layer "B.Cu") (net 29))
 (segment (start 58.4454 93.9383) (end 61.8843 93.9383) (width 0.2) (layer "B.Cu") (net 29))
 (segment (start 57.5817 94.802) (end 58.4454 93.9383) (width 0.2) (layer "B.Cu") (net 29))
 (segment (start 61.8843 93.9383) (end 64.4968 91.3258) (width 0.2) (layer "B.Cu") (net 29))
 (segment (start 64.5 71.05) (end 65.5478 72.0978) (width 0.2) (layer "B.Cu") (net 29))
 (segment (start 65.5478 72.0978) (end 69.7948 72.0978) (width 0.2) (layer "B.Cu") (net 29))
 (segment (start 64.4968 91.3258) (end 69.7948 91.3258) (width 0.2) (layer "B.Cu") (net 29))
 (segment (start 56.43 95.09) (end 57.5817 95.09) (width 0.2) (layer "B.Cu") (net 29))
 (segment (start 63.4716 63.6272) (end 63.4716 66.8716) (width 0.2) (layer "F.Cu") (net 10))
 (segment (start 63.4716 66.8716) (end 64.5 67.9) (width 0.2) (layer "F.Cu") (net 10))
 (via (at 63.4716 63.6272) (size 0.6) (drill 0.3) (layers "F.Cu" "B.Cu") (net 10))
 (segment (start 60.1217 64.61) (end 61.6921 63.0396) (width 0.2) (layer "B.Cu") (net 10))
 (segment (start 62.884 61.1603) (end 62.884 63.0396) (width 0.2) (layer "B.Cu") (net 10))
 (segment (start 62.884 63.0396) (end 63.4716 63.6272) (width 0.2) (layer "B.Cu") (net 10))
 (segment (start 61.6921 63.0396) (end 62.884 63.0396) (width 0.2) (layer "B.Cu") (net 10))
 (segment (start 58.97 64.61) (end 60.1217 64.61) (width 0.2) (layer "B.Cu") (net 10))
 (segment (start 75 53.5) (end 68.6413 59.8587) (width 0.2) (layer "B.Cu") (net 10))
 (segment (start 68.6413 59.8587) (end 64.1856 59.8587) (width 0.2) (layer "B.Cu") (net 10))
 (segment (start 64.1856 59.8587) (end 62.884 61.1603) (width 0.2) (layer "B.Cu") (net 10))
 (segment (start 56.7058 63.4583) (end 57.7 62.4641) (width 0.2) (layer "B.Cu") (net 12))
 (segment (start 55.2574 64.1027) (end 55.9018 63.4583) (width 0.2) (layer "B.Cu") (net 12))
 (segment (start 55.2289 69.2343) (end 56.1615 68.3017) (width 0.2) (layer "B.Cu") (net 12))
 (segment (start 57.7 62.4641) (end 57.7 61.6516) (width 0.2) (layer "B.Cu") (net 12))
 (segment (start 56.0464 70.96) (end 55.2289 70.1425) (width 0.2) (layer "B.Cu") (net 12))
 (segment (start 56.1421 65.9983) (end 55.2574 65.1136) (width 0.2) (layer "B.Cu") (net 12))
 (segment (start 58.5516 60.8) (end 59.3594 60.8) (width 0.2) (layer "B.Cu") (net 12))
 (segment (start 55.2574 65.1136) (end 55.2574 64.1027) (width 0.2) (layer "B.Cu") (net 12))
 (segment (start 63.7636 73.5) (end 61.2236 70.96) (width 0.2) (layer "B.Cu") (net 12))
 (segment (start 61.2236 70.96) (end 56.0464 70.96) (width 0.2) (layer "B.Cu") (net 12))
 (segment (start 59.3594 60.8) (end 64.5 55.6594) (width 0.2) (layer "B.Cu") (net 12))
 (segment (start 56.43 67.15) (end 56.43 68.3017) (width 0.2) (layer "B.Cu") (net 12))
 (segment (start 56.43 65.9983) (end 56.1421 65.9983) (width 0.2) (layer "B.Cu") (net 12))
 (segment (start 56.43 67.15) (end 56.43 65.9983) (width 0.2) (layer "B.Cu") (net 12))
 (segment (start 75 73.5) (end 63.7636 73.5) (width 0.2) (layer "B.Cu") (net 12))
 (segment (start 56.1615 68.3017) (end 56.43 68.3017) (width 0.2) (layer "B.Cu") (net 12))
 (segment (start 55.9018 63.4583) (end 56.7058 63.4583) (width 0.2) (layer "B.Cu") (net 12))
 (segment (start 55.2289 70.1425) (end 55.2289 69.2343) (width 0.2) (layer "B.Cu") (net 12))
 (segment (start 64.5 55.6594) (end 64.5 55.3) (width 0.2) (layer "B.Cu") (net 12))
 (segment (start 57.7 61.6516) (end 58.5516 60.8) (width 0.2) (layer "B.Cu") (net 12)))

